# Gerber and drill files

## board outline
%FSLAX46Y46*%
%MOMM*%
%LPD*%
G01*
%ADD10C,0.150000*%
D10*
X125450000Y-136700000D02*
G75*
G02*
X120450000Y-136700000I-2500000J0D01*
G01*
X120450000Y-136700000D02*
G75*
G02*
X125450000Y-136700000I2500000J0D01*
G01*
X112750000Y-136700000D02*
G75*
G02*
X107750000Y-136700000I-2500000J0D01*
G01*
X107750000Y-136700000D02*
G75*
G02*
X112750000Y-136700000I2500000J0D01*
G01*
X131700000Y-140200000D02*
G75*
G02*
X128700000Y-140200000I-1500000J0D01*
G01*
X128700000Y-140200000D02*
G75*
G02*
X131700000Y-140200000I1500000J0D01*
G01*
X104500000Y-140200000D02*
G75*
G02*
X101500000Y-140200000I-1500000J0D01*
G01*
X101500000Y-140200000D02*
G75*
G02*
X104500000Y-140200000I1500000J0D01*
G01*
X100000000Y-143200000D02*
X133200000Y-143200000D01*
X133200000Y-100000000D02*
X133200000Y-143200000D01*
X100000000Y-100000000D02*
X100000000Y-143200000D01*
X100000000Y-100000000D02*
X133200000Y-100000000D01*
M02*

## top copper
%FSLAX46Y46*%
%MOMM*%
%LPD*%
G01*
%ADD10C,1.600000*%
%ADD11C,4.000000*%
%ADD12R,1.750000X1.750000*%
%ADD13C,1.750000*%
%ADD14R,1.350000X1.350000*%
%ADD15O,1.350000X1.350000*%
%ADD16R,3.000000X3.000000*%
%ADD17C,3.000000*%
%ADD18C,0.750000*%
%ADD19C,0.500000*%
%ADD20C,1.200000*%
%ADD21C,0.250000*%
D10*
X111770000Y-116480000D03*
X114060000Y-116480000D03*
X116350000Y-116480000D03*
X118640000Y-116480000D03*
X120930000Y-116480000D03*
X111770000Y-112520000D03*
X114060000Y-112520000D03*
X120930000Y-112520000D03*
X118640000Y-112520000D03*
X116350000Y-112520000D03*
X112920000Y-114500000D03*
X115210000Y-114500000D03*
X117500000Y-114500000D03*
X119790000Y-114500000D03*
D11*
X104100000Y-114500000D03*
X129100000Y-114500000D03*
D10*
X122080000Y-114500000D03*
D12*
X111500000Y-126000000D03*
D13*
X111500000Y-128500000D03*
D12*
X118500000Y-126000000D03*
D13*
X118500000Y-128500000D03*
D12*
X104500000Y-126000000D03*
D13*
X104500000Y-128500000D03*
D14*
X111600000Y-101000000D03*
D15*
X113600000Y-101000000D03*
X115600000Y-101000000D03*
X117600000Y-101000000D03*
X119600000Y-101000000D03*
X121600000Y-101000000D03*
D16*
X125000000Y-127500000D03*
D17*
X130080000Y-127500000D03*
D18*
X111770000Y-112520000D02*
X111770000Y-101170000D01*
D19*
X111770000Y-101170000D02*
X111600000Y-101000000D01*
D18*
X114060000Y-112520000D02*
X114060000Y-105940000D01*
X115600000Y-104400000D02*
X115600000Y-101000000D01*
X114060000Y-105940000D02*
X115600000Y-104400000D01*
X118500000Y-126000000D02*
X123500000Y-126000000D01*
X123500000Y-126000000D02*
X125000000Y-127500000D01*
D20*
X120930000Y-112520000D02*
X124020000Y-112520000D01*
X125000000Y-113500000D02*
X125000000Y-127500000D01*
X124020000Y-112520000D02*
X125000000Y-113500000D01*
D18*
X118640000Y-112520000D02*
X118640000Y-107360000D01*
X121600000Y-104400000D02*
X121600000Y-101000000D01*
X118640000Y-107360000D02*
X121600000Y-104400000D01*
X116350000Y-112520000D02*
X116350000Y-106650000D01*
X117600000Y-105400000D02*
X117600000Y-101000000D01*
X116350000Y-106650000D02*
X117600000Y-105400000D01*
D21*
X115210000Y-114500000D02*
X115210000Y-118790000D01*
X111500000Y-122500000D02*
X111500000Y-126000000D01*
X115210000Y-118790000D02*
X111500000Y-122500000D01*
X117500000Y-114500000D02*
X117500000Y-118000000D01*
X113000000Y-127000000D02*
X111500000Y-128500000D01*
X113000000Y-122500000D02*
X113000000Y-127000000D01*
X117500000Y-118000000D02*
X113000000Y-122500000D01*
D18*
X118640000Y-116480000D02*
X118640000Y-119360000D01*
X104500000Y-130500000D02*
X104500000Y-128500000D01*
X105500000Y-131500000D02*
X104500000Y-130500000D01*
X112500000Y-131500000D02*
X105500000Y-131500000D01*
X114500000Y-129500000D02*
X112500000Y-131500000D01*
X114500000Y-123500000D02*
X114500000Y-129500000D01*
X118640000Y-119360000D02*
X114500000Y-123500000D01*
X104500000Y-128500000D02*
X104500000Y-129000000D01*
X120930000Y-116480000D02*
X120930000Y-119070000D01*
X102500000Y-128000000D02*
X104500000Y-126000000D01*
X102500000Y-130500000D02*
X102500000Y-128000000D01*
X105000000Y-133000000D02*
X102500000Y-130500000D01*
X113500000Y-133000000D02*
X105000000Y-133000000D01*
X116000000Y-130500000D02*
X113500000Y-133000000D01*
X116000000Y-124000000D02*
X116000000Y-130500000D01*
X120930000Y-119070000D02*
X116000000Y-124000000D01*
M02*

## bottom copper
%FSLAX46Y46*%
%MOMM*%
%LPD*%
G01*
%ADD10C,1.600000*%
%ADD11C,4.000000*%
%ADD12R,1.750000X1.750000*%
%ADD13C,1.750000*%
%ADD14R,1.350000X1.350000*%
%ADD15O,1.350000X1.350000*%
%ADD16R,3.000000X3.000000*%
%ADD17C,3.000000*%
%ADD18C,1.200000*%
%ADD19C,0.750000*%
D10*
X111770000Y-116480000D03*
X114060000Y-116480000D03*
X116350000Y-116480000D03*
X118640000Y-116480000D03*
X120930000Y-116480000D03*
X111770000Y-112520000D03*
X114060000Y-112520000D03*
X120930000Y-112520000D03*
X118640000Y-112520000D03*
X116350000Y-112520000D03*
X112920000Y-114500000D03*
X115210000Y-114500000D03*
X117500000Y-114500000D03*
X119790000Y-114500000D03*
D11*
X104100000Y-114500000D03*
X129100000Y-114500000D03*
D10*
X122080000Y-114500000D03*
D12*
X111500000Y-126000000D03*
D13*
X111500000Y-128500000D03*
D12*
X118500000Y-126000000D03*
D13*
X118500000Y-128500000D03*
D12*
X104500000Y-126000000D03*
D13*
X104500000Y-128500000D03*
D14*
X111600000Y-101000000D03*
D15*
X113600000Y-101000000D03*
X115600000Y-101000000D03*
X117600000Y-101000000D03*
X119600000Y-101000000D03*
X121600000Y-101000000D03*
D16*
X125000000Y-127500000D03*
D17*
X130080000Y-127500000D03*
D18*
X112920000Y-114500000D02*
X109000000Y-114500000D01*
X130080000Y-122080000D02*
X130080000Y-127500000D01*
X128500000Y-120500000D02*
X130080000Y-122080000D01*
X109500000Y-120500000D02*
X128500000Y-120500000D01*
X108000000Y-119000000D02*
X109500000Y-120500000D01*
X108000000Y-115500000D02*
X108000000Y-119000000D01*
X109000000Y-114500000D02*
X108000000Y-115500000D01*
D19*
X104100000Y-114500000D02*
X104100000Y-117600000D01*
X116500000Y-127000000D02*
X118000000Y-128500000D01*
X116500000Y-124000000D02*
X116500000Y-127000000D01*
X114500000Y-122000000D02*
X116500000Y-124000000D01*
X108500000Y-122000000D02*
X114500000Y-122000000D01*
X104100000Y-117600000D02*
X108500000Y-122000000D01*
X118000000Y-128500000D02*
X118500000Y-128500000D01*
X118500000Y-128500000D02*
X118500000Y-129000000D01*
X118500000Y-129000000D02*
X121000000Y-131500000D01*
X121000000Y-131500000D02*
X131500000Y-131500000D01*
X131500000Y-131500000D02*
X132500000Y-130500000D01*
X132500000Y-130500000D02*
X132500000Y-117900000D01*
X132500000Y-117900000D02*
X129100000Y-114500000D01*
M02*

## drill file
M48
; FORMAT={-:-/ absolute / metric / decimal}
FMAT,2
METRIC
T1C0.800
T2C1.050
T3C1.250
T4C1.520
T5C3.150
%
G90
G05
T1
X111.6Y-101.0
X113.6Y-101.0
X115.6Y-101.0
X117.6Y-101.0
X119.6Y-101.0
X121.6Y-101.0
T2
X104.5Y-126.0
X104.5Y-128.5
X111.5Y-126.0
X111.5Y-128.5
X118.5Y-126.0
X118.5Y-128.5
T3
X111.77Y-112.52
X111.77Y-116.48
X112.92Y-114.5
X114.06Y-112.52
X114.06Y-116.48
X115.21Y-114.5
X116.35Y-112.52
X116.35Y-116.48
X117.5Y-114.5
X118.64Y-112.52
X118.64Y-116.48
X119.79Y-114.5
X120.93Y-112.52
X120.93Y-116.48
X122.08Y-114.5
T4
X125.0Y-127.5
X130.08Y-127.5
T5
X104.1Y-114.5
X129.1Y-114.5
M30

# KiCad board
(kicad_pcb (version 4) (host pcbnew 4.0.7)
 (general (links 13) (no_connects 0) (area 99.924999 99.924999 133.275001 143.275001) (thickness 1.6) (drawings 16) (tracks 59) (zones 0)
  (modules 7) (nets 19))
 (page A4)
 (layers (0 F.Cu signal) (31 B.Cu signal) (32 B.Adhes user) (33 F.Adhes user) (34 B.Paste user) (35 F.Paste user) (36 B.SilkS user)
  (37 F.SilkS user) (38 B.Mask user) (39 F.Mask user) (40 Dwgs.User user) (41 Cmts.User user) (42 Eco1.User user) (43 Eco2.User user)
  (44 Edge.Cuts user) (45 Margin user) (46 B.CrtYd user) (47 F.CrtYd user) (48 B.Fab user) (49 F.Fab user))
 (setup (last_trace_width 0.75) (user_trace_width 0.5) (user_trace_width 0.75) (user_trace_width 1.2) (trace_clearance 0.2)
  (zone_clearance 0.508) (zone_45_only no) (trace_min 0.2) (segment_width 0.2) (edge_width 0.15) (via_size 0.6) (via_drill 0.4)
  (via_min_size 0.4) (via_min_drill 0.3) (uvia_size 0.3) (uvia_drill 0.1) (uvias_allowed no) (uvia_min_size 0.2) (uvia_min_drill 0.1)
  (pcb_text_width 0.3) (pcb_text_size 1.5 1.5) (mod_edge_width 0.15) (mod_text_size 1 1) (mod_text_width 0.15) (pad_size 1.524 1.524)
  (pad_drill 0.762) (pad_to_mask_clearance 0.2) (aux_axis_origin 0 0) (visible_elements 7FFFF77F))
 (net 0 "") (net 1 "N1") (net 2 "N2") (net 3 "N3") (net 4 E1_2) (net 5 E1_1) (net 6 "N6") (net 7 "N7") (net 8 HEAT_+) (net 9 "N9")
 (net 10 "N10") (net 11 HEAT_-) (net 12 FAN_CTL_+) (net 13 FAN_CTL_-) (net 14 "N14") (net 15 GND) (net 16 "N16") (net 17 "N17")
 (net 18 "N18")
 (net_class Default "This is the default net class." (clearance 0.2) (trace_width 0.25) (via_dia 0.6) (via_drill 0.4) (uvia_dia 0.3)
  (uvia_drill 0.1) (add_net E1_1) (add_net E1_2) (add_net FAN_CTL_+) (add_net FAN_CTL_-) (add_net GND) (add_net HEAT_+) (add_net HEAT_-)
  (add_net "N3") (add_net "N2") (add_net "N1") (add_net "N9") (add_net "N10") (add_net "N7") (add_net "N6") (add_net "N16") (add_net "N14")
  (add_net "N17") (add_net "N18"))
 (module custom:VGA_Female (layer F.Cu) (at 116.6 114.5)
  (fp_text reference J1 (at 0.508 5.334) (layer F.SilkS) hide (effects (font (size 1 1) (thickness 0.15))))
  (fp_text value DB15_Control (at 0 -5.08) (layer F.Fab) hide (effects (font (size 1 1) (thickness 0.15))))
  (pad 15 thru_hole circle (at -4.83 1.98) (size 1.6 1.6) (drill 1.25) (layers *.Cu *.Mask) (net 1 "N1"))
  (pad 14 thru_hole circle (at -2.54 1.98) (size 1.6 1.6) (drill 1.25) (layers *.Cu *.Mask) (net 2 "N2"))
  (pad 13 thru_hole circle (at -0.25 1.98) (size 1.6 1.6) (drill 1.25) (layers *.Cu *.Mask) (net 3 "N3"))
  (pad 12 thru_hole circle (at 2.04 1.98) (size 1.6 1.6) (drill 1.25) (layers *.Cu *.Mask) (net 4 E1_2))
  (pad 11 thru_hole circle (at 4.33 1.98) (size 1.6 1.6) (drill 1.25) (layers *.Cu *.Mask) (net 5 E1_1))
  (pad 5 thru_hole circle (at -4.83 -1.98) (size 1.6 1.6) (drill 1.25) (layers *.Cu *.Mask) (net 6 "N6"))
  (pad 4 thru_hole circle (at -2.54 -1.98) (size 1.6 1.6) (drill 1.25) (layers *.Cu *.Mask) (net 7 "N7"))
  (pad 1 thru_hole circle (at 4.33 -1.98) (size 1.6 1.6) (drill 1.25) (layers *.Cu *.Mask) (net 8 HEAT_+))
  (pad 2 thru_hole circle (at 2.04 -1.98) (size 1.6 1.6) (drill 1.25) (layers *.Cu *.Mask) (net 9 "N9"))
  (pad 3 thru_hole circle (at -0.25 -1.98) (size 1.6 1.6) (drill 1.25) (layers *.Cu *.Mask) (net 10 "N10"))
  (pad 10 thru_hole circle (at -3.68 0) (size 1.6 1.6) (drill 1.25) (layers *.Cu *.Mask) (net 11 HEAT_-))
  (pad 9 thru_hole circle (at -1.39 0) (size 1.6 1.6) (drill 1.25) (layers *.Cu *.Mask) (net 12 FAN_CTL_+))
  (pad 8 thru_hole circle (at 0.9 0) (size 1.6 1.6) (drill 1.25) (layers *.Cu *.Mask) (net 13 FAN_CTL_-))
  (pad 7 thru_hole circle (at 3.19 0) (size 1.6 1.6) (drill 1.25) (layers *.Cu *.Mask) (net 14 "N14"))
  (pad 0 thru_hole circle (at -12.5 0) (size 4 4) (drill 3.15) (layers *.Cu *.Mask) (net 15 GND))
  (pad 0 thru_hole circle (at 12.5 0) (size 4 4) (drill 3.15) (layers *.Cu *.Mask) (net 15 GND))
  (pad 6 thru_hole circle (at 5.48 0) (size 1.6 1.6) (drill 1.25) (layers *.Cu *.Mask) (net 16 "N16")))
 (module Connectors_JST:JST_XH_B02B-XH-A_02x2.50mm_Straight (layer F.Cu) (at 111.5 126 270)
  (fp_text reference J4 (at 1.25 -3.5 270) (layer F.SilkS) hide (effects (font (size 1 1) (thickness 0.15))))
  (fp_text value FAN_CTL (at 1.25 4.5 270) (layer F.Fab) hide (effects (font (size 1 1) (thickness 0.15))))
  (pad 1 thru_hole rect (at 0 0 270) (size 1.75 1.75) (drill 1.05) (layers *.Cu *.Mask) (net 12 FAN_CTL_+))
  (pad 2 thru_hole circle (at 2.5 0 270) (size 1.75 1.75) (drill 1.05) (layers *.Cu *.Mask) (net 13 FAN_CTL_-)))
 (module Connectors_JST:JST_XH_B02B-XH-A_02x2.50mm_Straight (layer F.Cu) (at 118.5 126 270)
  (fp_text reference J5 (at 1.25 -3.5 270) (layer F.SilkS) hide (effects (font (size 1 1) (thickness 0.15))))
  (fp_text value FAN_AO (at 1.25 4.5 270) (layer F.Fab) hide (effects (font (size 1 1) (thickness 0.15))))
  (pad 1 thru_hole rect (at 0 0 270) (size 1.75 1.75) (drill 1.05) (layers *.Cu *.Mask) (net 8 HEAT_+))
  (pad 2 thru_hole circle (at 2.5 0 270) (size 1.75 1.75) (drill 1.05) (layers *.Cu *.Mask) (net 15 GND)))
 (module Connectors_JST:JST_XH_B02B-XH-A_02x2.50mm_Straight (layer F.Cu) (at 104.5 126 270)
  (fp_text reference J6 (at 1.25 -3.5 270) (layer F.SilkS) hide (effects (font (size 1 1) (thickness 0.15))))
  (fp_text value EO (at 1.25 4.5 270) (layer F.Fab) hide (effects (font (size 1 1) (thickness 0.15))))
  (pad 1 thru_hole rect (at 0 0 270) (size 1.75 1.75) (drill 1.05) (layers *.Cu *.Mask) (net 5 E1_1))
  (pad 2 thru_hole circle (at 2.5 0 270) (size 1.75 1.75) (drill 1.05) (layers *.Cu *.Mask) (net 4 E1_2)))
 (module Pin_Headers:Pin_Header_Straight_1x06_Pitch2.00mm (layer F.Cu) (at 111.6 101 90)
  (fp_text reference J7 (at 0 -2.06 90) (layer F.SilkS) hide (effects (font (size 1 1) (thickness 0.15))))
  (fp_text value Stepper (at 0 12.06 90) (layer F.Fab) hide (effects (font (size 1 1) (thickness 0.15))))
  (pad 1 thru_hole rect (at 0 0 90) (size 1.35 1.35) (drill 0.8) (layers *.Cu *.Mask) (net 6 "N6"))
  (pad 2 thru_hole oval (at 0 2 90) (size 1.35 1.35) (drill 0.8) (layers *.Cu *.Mask) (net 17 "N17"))
  (pad 3 thru_hole oval (at 0 4 90) (size 1.35 1.35) (drill 0.8) (layers *.Cu *.Mask) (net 7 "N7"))
  (pad 4 thru_hole oval (at 0 6 90) (size 1.35 1.35) (drill 0.8) (layers *.Cu *.Mask) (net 10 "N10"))
  (pad 5 thru_hole oval (at 0 8 90) (size 1.35 1.35) (drill 0.8) (layers *.Cu *.Mask) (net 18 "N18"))
  (pad 6 thru_hole oval (at 0 10 90) (size 1.35 1.35) (drill 0.8) (layers *.Cu *.Mask) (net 9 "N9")))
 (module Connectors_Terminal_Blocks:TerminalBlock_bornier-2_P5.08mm (layer F.Cu) (at 125 127.5)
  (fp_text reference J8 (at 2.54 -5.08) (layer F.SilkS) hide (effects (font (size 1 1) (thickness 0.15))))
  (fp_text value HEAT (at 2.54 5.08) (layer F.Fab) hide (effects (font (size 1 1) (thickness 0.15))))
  (pad 1 thru_hole rect (at 0 0) (size 3 3) (drill 1.52) (layers *.Cu *.Mask) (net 8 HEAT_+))
  (pad 2 thru_hole circle (at 5.08 0) (size 3 3) (drill 1.52) (layers *.Cu *.Mask) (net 11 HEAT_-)))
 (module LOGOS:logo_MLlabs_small (layer B.Cu) (at 108.5 117.5 180)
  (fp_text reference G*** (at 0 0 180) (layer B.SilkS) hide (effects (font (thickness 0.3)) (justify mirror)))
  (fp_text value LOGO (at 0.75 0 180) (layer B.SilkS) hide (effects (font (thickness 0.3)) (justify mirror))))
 (gr_circle (center 122.95 136.7) (end 125.45 136.7) (layer Edge.Cuts) (width 0.15))
 (gr_circle (center 110.25 136.7) (end 112.75 136.7) (layer Edge.Cuts) (width 0.15))
 (gr_circle (center 130.2 140.2) (end 131.7 140.2) (layer Edge.Cuts) (width 0.15))
 (gr_circle (center 103 140.2) (end 104.5 140.2) (layer Edge.Cuts) (width 0.15))
 (gr_line (start 100 143.2) (end 133.2 143.2) (angle 90) (layer Edge.Cuts) (width 0.15))
 (gr_line (start 133.2 100) (end 133.2 143.2) (angle 90) (layer Edge.Cuts) (width 0.15))
 (gr_line (start 100 100) (end 100 143.2) (angle 90) (layer Edge.Cuts) (width 0.15))
 (gr_line (start 100 100) (end 133.2 100) (angle 90) (layer Edge.Cuts) (width 0.15))
 (segment (start 111.77 112.52) (end 111.77 101.17) (width 0.75) (layer F.Cu) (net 6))
 (segment (start 111.77 101.17) (end 111.6 101) (width 0.5) (layer F.Cu) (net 6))
 (segment (start 114.06 112.52) (end 114.06 105.94) (width 0.75) (layer F.Cu) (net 7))
 (segment (start 115.6 104.4) (end 115.6 101) (width 0.75) (layer F.Cu) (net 7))
 (segment (start 114.06 105.94) (end 115.6 104.4) (width 0.75) (layer F.Cu) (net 7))
 (segment (start 118.5 126) (end 123.5 126) (width 0.75) (layer F.Cu) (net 8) (status C00000))
 (segment (start 123.5 126) (end 125 127.5) (width 0.75) (layer F.Cu) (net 8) (status C00000))
 (segment (start 120.93 112.52) (end 124.02 112.52) (width 1.2) (layer F.Cu) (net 8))
 (segment (start 125 113.5) (end 125 127.5) (width 1.2) (layer F.Cu) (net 8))
 (segment (start 124.02 112.52) (end 125 113.5) (width 1.2) (layer F.Cu) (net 8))
 (segment (start 118.64 112.52) (end 118.64 107.36) (width 0.75) (layer F.Cu) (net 9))
 (segment (start 121.6 104.4) (end 121.6 101) (width 0.75) (layer F.Cu) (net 9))
 (segment (start 118.64 107.36) (end 121.6 104.4) (width 0.75) (layer F.Cu) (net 9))
 (segment (start 116.35 112.52) (end 116.35 106.65) (width 0.75) (layer F.Cu) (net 10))
 (segment (start 117.6 105.4) (end 117.6 101) (width 0.75) (layer F.Cu) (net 10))
 (segment (start 116.35 106.65) (end 117.6 105.4) (width 0.75) (layer F.Cu) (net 10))
 (segment (start 112.92 114.5) (end 109 114.5) (width 1.2) (layer B.Cu) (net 11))
 (segment (start 130.08 122.08) (end 130.08 127.5) (width 1.2) (layer B.Cu) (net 11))
 (segment (start 128.5 120.5) (end 130.08 122.08) (width 1.2) (layer B.Cu) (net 11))
 (segment (start 109.5 120.5) (end 128.5 120.5) (width 1.2) (layer B.Cu) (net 11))
 (segment (start 108 119) (end 109.5 120.5) (width 1.2) (layer B.Cu) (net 11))
 (segment (start 108 115.5) (end 108 119) (width 1.2) (layer B.Cu) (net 11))
 (segment (start 109 114.5) (end 108 115.5) (width 1.2) (layer B.Cu) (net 11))
 (segment (start 104.1 114.5) (end 104.1 117.6) (width 0.75) (layer B.Cu) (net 15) (status 400000))
 (segment (start 116.5 127) (end 118 128.5) (width 0.75) (layer B.Cu) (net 15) (status 800000))
 (segment (start 116.5 124) (end 116.5 127) (width 0.75) (layer B.Cu) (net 15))
 (segment (start 114.5 122) (end 116.5 124) (width 0.75) (layer B.Cu) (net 15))
 (segment (start 108.5 122) (end 114.5 122) (width 0.75) (layer B.Cu) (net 15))
 (segment (start 104.1 117.6) (end 108.5 122) (width 0.75) (layer B.Cu) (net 15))
 (segment (start 118 128.5) (end 118.5 128.5) (width 0.75) (layer B.Cu) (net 15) (status C00000))
 (segment (start 118.5 128.5) (end 118.5 129) (width 0.75) (layer B.Cu) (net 15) (status C00000))
 (segment (start 118.5 129) (end 121 131.5) (width 0.75) (layer B.Cu) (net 15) (status 400000))
 (segment (start 121 131.5) (end 131.5 131.5) (width 0.75) (layer B.Cu) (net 15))
 (segment (start 131.5 131.5) (end 132.5 130.5) (width 0.75) (layer B.Cu) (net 15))
 (segment (start 132.5 130.5) (end 132.5 117.9) (width 0.75) (layer B.Cu) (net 15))
 (segment (start 132.5 117.9) (end 129.1 114.5) (width 0.75) (layer B.Cu) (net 15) (status 800000))
 (segment (start 115.21 114.5) (end 115.21 118.79) (width 0.25) (layer F.Cu) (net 12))
 (segment (start 111.5 122.5) (end 111.5 126) (width 0.25) (layer F.Cu) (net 12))
 (segment (start 115.21 118.79) (end 111.5 122.5) (width 0.25) (layer F.Cu) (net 12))
 (segment (start 117.5 114.5) (end 117.5 118) (width 0.25) (layer F.Cu) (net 13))
 (segment (start 113 127) (end 111.5 128.5) (width 0.25) (layer F.Cu) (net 13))
 (segment (start 113 122.5) (end 113 127) (width 0.25) (layer F.Cu) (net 13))
 (segment (start 117.5 118) (end 113 122.5) (width 0.25) (layer F.Cu) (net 13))
 (segment (start 118.64 116.48) (end 118.64 119.36) (width 0.75) (layer F.Cu) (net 4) (status 400000))
 (segment (start 104.5 130.5) (end 104.5 128.5) (width 0.75) (layer F.Cu) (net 4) (status 800000))
 (segment (start 105.5 131.5) (end 104.5 130.5) (width 0.75) (layer F.Cu) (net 4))
 (segment (start 112.5 131.5) (end 105.5 131.5) (width 0.75) (layer F.Cu) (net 4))
 (segment (start 114.5 129.5) (end 112.5 131.5) (width 0.75) (layer F.Cu) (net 4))
 (segment (start 114.5 123.5) (end 114.5 129.5) (width 0.75) (layer F.Cu) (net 4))
 (segment (start 118.64 119.36) (end 114.5 123.5) (width 0.75) (layer F.Cu) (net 4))
 (segment (start 104.5 128.5) (end 104.5 129) (width 0.75) (layer F.Cu) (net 4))
 (segment (start 120.93 116.48) (end 120.93 119.07) (width 0.75) (layer F.Cu) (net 5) (status 400000))
 (segment (start 102.5 128) (end 104.5 126) (width 0.75) (layer F.Cu) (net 5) (status 800000))
 (segment (start 102.5 130.5) (end 102.5 128) (width 0.75) (layer F.Cu) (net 5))
 (segment (start 105 133) (end 102.5 130.5) (width 0.75) (layer F.Cu) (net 5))
 (segment (start 113.5 133) (end 105 133) (width 0.75) (layer F.Cu) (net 5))
 (segment (start 116 130.5) (end 113.5 133) (width 0.75) (layer F.Cu) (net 5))
 (segment (start 116 124) (end 116 130.5) (width 0.75) (layer F.Cu) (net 5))
 (segment (start 120.93 119.07) (end 116 124) (width 0.75) (layer F.Cu) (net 5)))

